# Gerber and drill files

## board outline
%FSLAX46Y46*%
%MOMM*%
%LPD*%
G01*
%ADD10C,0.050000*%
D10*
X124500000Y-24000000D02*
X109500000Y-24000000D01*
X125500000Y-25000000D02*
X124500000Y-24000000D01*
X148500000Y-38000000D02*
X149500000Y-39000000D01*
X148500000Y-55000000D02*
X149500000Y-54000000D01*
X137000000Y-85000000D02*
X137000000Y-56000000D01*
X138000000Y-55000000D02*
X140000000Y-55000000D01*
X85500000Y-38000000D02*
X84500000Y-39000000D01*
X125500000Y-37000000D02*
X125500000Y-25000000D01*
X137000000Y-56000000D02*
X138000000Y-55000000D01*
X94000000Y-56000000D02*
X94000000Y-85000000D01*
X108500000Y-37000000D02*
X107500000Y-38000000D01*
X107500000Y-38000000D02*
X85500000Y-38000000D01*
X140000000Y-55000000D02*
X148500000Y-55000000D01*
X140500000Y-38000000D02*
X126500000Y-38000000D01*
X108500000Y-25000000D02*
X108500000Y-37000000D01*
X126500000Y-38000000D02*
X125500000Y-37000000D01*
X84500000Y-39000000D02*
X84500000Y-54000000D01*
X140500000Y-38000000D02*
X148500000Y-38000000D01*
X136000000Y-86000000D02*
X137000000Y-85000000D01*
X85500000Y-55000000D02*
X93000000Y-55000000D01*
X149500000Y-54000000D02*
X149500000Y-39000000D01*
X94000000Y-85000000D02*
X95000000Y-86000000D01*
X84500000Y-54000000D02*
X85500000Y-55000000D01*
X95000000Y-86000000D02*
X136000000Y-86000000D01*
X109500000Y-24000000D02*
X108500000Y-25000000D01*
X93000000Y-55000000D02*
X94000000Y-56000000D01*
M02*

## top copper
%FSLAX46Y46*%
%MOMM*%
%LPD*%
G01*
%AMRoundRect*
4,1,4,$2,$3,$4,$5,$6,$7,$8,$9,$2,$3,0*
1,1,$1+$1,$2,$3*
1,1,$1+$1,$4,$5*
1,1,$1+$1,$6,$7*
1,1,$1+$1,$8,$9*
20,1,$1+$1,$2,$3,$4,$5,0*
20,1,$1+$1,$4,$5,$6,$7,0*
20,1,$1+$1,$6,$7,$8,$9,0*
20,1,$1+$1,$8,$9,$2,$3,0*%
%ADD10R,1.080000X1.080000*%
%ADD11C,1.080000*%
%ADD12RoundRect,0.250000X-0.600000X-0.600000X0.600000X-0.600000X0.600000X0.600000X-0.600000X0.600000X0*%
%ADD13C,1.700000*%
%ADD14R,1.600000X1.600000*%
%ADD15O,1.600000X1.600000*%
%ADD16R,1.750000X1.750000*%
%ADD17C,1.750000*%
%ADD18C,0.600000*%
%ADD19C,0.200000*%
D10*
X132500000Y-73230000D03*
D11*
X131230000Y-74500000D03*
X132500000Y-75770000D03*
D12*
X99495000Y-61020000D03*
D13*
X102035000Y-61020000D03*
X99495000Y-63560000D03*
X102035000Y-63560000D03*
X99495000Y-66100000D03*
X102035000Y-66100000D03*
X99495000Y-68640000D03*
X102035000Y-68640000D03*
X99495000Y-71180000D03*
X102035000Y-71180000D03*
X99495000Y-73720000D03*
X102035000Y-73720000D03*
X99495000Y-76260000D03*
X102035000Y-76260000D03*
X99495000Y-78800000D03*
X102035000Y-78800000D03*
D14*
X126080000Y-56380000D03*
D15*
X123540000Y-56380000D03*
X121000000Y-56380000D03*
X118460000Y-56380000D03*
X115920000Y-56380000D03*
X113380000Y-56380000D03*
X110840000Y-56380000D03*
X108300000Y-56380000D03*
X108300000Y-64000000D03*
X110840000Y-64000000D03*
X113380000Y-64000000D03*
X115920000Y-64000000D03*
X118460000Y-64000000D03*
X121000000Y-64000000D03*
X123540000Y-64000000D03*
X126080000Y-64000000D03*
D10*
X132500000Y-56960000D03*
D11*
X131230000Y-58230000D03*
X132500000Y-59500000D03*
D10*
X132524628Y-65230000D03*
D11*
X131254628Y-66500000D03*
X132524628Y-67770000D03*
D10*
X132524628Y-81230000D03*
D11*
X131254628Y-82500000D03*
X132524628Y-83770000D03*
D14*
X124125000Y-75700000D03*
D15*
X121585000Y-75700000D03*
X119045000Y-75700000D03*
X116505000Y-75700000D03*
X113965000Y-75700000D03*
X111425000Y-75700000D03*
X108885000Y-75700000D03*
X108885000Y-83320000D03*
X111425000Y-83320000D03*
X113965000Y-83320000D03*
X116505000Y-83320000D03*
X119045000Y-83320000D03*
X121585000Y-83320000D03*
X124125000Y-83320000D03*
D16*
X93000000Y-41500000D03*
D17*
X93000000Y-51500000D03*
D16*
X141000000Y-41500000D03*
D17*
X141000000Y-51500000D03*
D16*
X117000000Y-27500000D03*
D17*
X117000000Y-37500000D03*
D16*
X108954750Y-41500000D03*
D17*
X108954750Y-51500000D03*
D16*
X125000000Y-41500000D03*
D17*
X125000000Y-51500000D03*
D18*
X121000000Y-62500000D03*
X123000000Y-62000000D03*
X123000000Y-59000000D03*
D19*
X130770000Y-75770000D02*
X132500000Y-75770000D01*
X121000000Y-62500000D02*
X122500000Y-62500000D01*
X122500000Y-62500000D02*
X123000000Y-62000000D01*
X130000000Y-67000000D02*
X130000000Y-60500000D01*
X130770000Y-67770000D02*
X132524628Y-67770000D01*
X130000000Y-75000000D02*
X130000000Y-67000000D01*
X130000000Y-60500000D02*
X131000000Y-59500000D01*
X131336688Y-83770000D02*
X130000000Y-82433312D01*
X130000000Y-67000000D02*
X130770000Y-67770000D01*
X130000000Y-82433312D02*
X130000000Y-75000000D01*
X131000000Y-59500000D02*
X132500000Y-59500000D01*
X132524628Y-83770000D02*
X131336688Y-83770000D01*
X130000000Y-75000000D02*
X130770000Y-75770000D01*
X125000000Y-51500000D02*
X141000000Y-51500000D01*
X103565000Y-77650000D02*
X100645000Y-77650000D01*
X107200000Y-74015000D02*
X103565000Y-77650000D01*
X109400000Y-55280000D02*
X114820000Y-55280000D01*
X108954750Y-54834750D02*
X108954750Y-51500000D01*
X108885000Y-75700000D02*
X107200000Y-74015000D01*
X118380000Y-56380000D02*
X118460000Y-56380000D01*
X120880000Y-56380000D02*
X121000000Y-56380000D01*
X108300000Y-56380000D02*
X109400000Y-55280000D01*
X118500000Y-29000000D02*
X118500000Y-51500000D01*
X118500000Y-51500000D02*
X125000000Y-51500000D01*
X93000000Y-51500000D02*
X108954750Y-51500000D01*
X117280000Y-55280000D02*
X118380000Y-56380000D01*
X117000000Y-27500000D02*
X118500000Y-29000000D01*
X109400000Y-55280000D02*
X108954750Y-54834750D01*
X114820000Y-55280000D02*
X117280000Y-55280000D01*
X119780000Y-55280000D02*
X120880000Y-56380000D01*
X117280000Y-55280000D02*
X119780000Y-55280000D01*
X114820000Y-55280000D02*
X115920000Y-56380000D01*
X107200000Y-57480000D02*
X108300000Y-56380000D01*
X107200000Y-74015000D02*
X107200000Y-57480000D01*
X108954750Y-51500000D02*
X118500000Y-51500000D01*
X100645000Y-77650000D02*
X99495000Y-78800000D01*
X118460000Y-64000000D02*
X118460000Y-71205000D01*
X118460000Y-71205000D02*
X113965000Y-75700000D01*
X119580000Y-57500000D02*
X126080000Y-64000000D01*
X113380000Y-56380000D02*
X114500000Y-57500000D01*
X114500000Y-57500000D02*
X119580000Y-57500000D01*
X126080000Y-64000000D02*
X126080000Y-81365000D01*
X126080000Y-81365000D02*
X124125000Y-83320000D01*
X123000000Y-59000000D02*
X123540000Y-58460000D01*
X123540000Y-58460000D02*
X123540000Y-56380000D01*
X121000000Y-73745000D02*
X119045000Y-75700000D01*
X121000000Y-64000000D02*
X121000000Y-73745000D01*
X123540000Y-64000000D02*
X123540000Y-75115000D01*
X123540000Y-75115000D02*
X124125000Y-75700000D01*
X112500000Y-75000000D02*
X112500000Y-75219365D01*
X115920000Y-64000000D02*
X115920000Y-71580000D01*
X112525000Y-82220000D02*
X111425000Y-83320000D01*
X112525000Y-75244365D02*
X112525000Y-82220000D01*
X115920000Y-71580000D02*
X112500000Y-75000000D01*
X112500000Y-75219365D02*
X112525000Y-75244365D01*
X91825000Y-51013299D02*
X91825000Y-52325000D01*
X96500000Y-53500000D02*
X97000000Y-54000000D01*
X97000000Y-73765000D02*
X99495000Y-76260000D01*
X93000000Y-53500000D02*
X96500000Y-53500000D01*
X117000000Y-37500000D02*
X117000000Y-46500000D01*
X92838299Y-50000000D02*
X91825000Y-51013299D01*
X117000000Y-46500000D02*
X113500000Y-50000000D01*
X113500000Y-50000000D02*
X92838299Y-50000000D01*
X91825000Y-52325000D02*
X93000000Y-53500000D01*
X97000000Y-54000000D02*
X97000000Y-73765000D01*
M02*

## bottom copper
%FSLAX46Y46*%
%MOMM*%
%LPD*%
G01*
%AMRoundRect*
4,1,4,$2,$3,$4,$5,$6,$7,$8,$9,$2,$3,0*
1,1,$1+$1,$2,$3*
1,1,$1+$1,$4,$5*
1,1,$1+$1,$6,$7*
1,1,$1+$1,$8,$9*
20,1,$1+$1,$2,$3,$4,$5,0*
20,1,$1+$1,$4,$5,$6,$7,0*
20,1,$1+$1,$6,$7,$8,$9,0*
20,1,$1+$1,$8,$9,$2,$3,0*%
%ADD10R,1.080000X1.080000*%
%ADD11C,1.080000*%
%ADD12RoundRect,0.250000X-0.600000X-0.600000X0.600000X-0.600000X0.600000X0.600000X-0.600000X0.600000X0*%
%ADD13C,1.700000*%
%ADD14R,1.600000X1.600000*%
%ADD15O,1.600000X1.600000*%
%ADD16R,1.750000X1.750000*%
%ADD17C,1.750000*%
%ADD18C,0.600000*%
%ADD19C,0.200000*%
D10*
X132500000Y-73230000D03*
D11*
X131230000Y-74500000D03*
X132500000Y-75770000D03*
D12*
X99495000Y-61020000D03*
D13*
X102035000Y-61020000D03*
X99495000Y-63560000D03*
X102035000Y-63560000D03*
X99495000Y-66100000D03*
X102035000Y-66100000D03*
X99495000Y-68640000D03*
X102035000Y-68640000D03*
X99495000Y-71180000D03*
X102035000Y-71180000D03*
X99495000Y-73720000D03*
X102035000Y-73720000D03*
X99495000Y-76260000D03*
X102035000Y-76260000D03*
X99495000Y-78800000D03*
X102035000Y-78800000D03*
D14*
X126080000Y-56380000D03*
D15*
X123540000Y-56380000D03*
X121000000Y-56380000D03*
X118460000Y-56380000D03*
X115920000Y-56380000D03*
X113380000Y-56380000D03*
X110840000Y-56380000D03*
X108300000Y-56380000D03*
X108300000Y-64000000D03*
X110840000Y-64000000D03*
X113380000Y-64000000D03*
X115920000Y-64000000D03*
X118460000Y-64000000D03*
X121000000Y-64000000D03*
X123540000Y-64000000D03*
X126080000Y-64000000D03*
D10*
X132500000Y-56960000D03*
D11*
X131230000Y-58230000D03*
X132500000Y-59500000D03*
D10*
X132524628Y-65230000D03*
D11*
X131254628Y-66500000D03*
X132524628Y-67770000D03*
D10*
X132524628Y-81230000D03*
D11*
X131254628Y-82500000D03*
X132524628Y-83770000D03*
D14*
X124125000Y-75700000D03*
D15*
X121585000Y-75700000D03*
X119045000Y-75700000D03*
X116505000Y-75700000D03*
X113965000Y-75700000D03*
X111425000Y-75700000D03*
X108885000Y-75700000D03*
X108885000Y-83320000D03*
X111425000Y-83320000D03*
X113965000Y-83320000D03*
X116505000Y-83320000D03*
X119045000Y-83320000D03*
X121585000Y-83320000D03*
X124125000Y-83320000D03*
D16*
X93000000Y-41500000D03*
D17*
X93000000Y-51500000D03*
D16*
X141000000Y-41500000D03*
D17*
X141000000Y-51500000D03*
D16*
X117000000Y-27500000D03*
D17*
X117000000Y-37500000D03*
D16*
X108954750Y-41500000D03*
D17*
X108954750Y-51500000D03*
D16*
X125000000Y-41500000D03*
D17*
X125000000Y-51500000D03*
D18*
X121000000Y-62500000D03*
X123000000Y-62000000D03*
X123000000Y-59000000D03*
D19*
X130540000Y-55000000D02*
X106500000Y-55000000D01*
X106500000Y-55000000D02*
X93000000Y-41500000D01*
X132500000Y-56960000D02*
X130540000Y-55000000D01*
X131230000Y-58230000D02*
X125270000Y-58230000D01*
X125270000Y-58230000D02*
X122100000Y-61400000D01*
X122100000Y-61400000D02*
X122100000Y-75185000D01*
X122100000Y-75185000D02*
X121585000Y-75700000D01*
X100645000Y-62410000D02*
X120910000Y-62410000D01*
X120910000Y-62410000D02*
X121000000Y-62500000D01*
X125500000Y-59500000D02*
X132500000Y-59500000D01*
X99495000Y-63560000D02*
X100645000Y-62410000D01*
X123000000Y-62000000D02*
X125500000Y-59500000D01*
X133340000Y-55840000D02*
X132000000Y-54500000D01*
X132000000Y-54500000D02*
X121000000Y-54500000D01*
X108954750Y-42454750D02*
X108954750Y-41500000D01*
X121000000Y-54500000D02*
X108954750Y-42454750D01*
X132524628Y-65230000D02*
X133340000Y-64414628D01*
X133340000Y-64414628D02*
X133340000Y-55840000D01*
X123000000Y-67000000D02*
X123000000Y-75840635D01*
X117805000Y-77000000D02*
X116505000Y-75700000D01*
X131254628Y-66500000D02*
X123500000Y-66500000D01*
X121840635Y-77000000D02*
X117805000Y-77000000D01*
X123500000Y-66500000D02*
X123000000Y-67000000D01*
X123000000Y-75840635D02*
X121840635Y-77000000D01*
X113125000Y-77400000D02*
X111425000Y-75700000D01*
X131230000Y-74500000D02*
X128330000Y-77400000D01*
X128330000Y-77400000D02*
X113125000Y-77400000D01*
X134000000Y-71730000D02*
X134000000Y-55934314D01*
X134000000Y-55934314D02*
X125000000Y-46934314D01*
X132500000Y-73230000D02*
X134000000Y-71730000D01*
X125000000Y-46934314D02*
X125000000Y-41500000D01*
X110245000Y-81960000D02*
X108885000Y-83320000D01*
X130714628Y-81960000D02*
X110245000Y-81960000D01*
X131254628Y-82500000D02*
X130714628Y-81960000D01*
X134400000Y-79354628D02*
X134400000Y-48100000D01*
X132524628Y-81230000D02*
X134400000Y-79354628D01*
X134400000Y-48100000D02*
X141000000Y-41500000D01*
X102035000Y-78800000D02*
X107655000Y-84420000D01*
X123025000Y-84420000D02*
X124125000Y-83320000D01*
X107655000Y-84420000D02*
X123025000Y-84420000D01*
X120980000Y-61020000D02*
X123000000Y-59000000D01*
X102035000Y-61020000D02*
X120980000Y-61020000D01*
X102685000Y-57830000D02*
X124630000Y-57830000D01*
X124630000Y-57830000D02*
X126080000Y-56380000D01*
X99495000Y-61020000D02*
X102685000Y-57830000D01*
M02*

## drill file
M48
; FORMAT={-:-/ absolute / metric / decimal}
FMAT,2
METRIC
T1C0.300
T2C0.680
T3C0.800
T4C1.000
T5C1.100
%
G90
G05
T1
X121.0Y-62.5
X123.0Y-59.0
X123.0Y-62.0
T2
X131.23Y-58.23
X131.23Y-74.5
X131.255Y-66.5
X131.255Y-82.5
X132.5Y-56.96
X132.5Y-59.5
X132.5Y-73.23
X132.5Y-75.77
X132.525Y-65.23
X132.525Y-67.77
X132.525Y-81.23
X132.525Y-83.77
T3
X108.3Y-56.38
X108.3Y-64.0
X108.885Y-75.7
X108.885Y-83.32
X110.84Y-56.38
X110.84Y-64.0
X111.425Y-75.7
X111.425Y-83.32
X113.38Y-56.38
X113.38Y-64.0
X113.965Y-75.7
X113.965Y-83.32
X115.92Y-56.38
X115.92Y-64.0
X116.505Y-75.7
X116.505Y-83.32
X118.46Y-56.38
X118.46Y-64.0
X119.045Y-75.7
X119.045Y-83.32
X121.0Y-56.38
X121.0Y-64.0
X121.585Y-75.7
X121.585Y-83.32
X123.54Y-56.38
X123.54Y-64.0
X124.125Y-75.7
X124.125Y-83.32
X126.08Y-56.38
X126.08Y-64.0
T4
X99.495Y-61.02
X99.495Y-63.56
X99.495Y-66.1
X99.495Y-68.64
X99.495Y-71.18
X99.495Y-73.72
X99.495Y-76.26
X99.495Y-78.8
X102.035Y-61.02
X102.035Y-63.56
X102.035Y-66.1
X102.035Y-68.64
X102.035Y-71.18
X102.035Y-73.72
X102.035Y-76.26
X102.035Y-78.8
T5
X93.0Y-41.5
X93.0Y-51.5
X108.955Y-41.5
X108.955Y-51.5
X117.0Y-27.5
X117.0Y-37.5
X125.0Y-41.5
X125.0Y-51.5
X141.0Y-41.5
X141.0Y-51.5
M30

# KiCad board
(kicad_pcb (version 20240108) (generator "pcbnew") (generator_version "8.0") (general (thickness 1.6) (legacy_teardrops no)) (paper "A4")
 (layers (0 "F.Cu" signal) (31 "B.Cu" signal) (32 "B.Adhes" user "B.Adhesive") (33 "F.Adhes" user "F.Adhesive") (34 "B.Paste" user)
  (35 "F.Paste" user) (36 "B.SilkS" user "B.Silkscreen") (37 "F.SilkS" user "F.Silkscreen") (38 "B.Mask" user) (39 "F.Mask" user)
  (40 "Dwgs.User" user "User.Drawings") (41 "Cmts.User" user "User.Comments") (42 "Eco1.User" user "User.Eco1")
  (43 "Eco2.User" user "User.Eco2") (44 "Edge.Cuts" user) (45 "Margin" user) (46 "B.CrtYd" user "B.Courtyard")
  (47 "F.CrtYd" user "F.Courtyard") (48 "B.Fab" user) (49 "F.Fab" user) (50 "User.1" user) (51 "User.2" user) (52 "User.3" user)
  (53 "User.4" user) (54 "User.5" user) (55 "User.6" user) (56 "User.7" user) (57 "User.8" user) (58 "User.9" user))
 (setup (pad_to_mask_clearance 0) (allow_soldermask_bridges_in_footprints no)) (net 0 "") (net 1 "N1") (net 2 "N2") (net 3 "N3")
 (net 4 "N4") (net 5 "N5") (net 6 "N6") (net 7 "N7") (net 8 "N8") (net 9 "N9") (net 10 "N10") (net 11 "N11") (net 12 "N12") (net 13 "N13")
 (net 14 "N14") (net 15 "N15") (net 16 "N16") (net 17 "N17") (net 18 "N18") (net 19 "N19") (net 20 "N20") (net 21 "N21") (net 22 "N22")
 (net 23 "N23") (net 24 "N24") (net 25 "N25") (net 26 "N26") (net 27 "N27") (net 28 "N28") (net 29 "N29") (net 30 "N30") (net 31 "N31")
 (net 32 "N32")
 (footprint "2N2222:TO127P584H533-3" (layer "F.Cu") (at 132.5 74.5 -90)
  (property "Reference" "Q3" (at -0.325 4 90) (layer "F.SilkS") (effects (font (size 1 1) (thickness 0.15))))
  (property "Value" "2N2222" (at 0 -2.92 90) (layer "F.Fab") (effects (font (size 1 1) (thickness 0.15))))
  (pad "1" thru_hole rect (at -1.27 0 270) (size 1.08 1.08) (drill 0.68) (layers "*.Cu" "*.Mask") (remove_unused_layers no) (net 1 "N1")
   (solder_mask_margin 0.102))
  (pad "2" thru_hole circle (at 0 1.27 270) (size 1.08 1.08) (drill 0.68) (layers "*.Cu" "*.Mask") (remove_unused_layers no) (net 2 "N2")
   (solder_mask_margin 0.102))
  (pad "3" thru_hole circle (at 1.27 0 267) (size 1.08 1.08) (drill 0.68) (layers "*.Cu" "*.Mask") (remove_unused_layers no) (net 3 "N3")
   (solder_mask_margin 0.102)))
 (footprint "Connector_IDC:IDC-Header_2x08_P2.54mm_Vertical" (layer "F.Cu") (at 99.495 61.02)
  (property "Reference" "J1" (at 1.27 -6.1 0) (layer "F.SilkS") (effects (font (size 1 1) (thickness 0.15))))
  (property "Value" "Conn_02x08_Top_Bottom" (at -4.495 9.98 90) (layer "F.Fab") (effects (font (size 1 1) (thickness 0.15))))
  (pad "1" thru_hole roundrect (at 0 0) (size 1.7 1.7) (drill 1) (layers "*.Cu" "*.Mask") (remove_unused_layers no)
   (roundrect_rratio 0.147059) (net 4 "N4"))
  (pad "2" thru_hole circle (at 2.54 0) (size 1.7 1.7) (drill 1) (layers "*.Cu" "*.Mask") (remove_unused_layers no) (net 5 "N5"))
  (pad "3" thru_hole circle (at 0 2.54) (size 1.7 1.7) (drill 1) (layers "*.Cu" "*.Mask") (remove_unused_layers no) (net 3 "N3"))
  (pad "4" thru_hole circle (at 2.54 2.54) (size 1.7 1.7) (drill 1) (layers "*.Cu" "*.Mask") (remove_unused_layers no) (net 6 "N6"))
  (pad "5" thru_hole circle (at 0 5.08) (size 1.7 1.7) (drill 1) (layers "*.Cu" "*.Mask") (remove_unused_layers no) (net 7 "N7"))
  (pad "6" thru_hole circle (at 2.54 5.08) (size 1.7 1.7) (drill 1) (layers "*.Cu" "*.Mask") (remove_unused_layers no) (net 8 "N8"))
  (pad "7" thru_hole circle (at 0 7.62) (size 1.7 1.7) (drill 1) (layers "*.Cu" "*.Mask") (remove_unused_layers no) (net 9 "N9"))
  (pad "8" thru_hole circle (at 2.54 7.62) (size 1.7 1.7) (drill 1) (layers "*.Cu" "*.Mask") (remove_unused_layers no) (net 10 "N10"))
  (pad "9" thru_hole circle (at 0 10.16) (size 1.7 1.7) (drill 1) (layers "*.Cu" "*.Mask") (remove_unused_layers no) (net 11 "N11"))
  (pad "10" thru_hole circle (at 2.54 10.16) (size 1.7 1.7) (drill 1) (layers "*.Cu" "*.Mask") (remove_unused_layers no) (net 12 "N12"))
  (pad "11" thru_hole circle (at 0 12.7) (size 1.7 1.7) (drill 1) (layers "*.Cu" "*.Mask") (remove_unused_layers no) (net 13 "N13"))
  (pad "12" thru_hole circle (at 2.54 12.7) (size 1.7 1.7) (drill 1) (layers "*.Cu" "*.Mask") (remove_unused_layers no) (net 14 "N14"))
  (pad "13" thru_hole circle (at 0 15.24) (size 1.7 1.7) (drill 1) (layers "*.Cu" "*.Mask") (remove_unused_layers no) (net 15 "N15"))
  (pad "14" thru_hole circle (at 2.54 15.24) (size 1.7 1.7) (drill 1) (layers "*.Cu" "*.Mask") (remove_unused_layers no) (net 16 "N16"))
  (pad "15" thru_hole circle (at 0 17.78) (size 1.7 1.7) (drill 1) (layers "*.Cu" "*.Mask") (remove_unused_layers no) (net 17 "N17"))
  (pad "16" thru_hole circle (at 2.54 17.78) (size 1.7 1.7) (drill 1) (layers "*.Cu" "*.Mask") (remove_unused_layers no) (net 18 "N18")))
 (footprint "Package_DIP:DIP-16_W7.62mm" (layer "F.Cu") (at 126.08 56.38 -90)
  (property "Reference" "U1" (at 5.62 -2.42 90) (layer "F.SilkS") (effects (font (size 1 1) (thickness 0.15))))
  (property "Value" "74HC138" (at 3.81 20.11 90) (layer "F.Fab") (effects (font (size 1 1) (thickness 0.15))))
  (pad "1" thru_hole rect (at 0 0 270) (size 1.6 1.6) (drill 0.8) (layers "*.Cu" "*.Mask") (remove_unused_layers no) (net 4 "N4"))
  (pad "2" thru_hole oval (at 0 2.54 270) (size 1.6 1.6) (drill 0.8) (layers "*.Cu" "*.Mask") (remove_unused_layers no) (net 5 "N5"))
  (pad "3" thru_hole oval (at 0 5.08 270) (size 1.6 1.6) (drill 0.8) (layers "*.Cu" "*.Mask") (remove_unused_layers no) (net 17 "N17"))
  (pad "4" thru_hole oval (at 0 7.62 270) (size 1.6 1.6) (drill 0.8) (layers "*.Cu" "*.Mask") (remove_unused_layers no) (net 17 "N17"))
  (pad "5" thru_hole oval (at 0 10.16 270) (size 1.6 1.6) (drill 0.8) (layers "*.Cu" "*.Mask") (remove_unused_layers no) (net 17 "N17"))
  (pad "6" thru_hole oval (at 0 12.7 270) (size 1.6 1.6) (drill 0.8) (layers "*.Cu" "*.Mask") (remove_unused_layers no) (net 18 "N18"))
  (pad "7" thru_hole oval (at 0 15.24 270) (size 1.6 1.6) (drill 0.8) (layers "*.Cu" "*.Mask") (remove_unused_layers no) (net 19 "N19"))
  (pad "8" thru_hole oval (at 0 17.78 270) (size 1.6 1.6) (drill 0.8) (layers "*.Cu" "*.Mask") (remove_unused_layers no) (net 17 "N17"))
  (pad "9" thru_hole oval (at 7.62 17.78 270) (size 1.6 1.6) (drill 0.8) (layers "*.Cu" "*.Mask") (remove_unused_layers no) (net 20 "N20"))
  (pad "10" thru_hole oval (at 7.62 15.24 270) (size 1.6 1.6) (drill 0.8) (layers "*.Cu" "*.Mask") (remove_unused_layers no) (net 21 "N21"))
  (pad "11" thru_hole oval (at 7.62 12.7 270) (size 1.6 1.6) (drill 0.8) (layers "*.Cu" "*.Mask") (remove_unused_layers no) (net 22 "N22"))
  (pad "12" thru_hole oval (at 7.62 10.16 270) (size 1.6 1.6) (drill 0.8) (layers "*.Cu" "*.Mask") (remove_unused_layers no) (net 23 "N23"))
  (pad "13" thru_hole oval (at 7.62 7.62 270) (size 1.6 1.6) (drill 0.8) (layers "*.Cu" "*.Mask") (remove_unused_layers no) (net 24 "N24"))
  (pad "14" thru_hole oval (at 7.62 5.08 270) (size 1.6 1.6) (drill 0.8) (layers "*.Cu" "*.Mask") (remove_unused_layers no) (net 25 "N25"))
  (pad "15" thru_hole oval (at 7.62 2.54 270) (size 1.6 1.6) (drill 0.8) (layers "*.Cu" "*.Mask") (remove_unused_layers no) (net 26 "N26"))
  (pad "16" thru_hole oval (at 7.62 0 270) (size 1.6 1.6) (drill 0.8) (layers "*.Cu" "*.Mask") (remove_unused_layers no) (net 18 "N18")))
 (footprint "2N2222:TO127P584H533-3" (layer "F.Cu") (at 132.5 58.23 -90)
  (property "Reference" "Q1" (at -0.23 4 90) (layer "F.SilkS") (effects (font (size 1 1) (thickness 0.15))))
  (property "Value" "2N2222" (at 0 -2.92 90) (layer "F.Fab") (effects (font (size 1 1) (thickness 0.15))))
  (pad "1" thru_hole rect (at -1.27 0 270) (size 1.08 1.08) (drill 0.68) (layers "*.Cu" "*.Mask") (remove_unused_layers no) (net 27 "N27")
   (solder_mask_margin 0.102))
  (pad "2" thru_hole circle (at 0 1.27 270) (size 1.08 1.08) (drill 0.68) (layers "*.Cu" "*.Mask") (remove_unused_layers no) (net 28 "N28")
   (solder_mask_margin 0.102))
  (pad "3" thru_hole circle (at 1.27 0 267) (size 1.08 1.08) (drill 0.68) (layers "*.Cu" "*.Mask") (remove_unused_layers no) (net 3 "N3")
   (solder_mask_margin 0.102)))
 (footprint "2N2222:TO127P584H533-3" (layer "F.Cu") (at 132.524628 66.5 -90)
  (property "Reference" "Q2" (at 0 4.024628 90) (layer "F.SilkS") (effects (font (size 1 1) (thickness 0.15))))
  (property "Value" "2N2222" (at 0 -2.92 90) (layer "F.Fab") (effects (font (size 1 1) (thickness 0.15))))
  (pad "1" thru_hole rect (at -1.27 0 270) (size 1.08 1.08) (drill 0.68) (layers "*.Cu" "*.Mask") (remove_unused_layers no) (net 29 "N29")
   (solder_mask_margin 0.102))
  (pad "2" thru_hole circle (at 0 1.27 270) (size 1.08 1.08) (drill 0.68) (layers "*.Cu" "*.Mask") (remove_unused_layers no) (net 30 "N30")
   (solder_mask_margin 0.102))
  (pad "3" thru_hole circle (at 1.27 0 267) (size 1.08 1.08) (drill 0.68) (layers "*.Cu" "*.Mask") (remove_unused_layers no) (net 3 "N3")
   (solder_mask_margin 0.102)))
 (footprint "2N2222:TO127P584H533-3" (layer "F.Cu") (at 132.524628 82.5 -90)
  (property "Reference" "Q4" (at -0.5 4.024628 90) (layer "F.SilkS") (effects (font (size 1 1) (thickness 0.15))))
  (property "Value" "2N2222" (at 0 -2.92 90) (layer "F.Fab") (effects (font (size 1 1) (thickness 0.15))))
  (pad "1" thru_hole rect (at -1.27 0 270) (size 1.08 1.08) (drill 0.68) (layers "*.Cu" "*.Mask") (remove_unused_layers no) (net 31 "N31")
   (solder_mask_margin 0.102))
  (pad "2" thru_hole circle (at 0 1.27 270) (size 1.08 1.08) (drill 0.68) (layers "*.Cu" "*.Mask") (remove_unused_layers no) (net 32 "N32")
   (solder_mask_margin 0.102))
  (pad "3" thru_hole circle (at 1.27 0 267) (size 1.08 1.08) (drill 0.68) (layers "*.Cu" "*.Mask") (remove_unused_layers no) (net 3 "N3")
   (solder_mask_margin 0.102)))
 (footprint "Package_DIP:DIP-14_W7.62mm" (layer "F.Cu") (at 124.125 75.7 -90)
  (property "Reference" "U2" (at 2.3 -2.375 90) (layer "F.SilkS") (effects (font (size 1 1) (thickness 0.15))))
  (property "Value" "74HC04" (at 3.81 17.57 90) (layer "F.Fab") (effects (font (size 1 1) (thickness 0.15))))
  (pad "1" thru_hole rect (at 0 0 270) (size 1.6 1.6) (drill 0.8) (layers "*.Cu" "*.Mask") (remove_unused_layers no) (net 26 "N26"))
  (pad "2" thru_hole oval (at 0 2.54 270) (size 1.6 1.6) (drill 0.8) (layers "*.Cu" "*.Mask") (remove_unused_layers no) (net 28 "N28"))
  (pad "3" thru_hole oval (at 0 5.08 270) (size 1.6 1.6) (drill 0.8) (layers "*.Cu" "*.Mask") (remove_unused_layers no) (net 25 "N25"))
  (pad "4" thru_hole oval (at 0 7.62 270) (size 1.6 1.6) (drill 0.8) (layers "*.Cu" "*.Mask") (remove_unused_layers no) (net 30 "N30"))
  (pad "5" thru_hole oval (at 0 10.16 270) (size 1.6 1.6) (drill 0.8) (layers "*.Cu" "*.Mask") (remove_unused_layers no) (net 24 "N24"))
  (pad "6" thru_hole oval (at 0 12.7 270) (size 1.6 1.6) (drill 0.8) (layers "*.Cu" "*.Mask") (remove_unused_layers no) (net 2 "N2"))
  (pad "7" thru_hole oval (at 0 15.24 270) (size 1.6 1.6) (drill 0.8) (layers "*.Cu" "*.Mask") (remove_unused_layers no) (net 17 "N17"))
  (pad "8" thru_hole oval (at 7.62 15.24 270) (size 1.6 1.6) (drill 0.8) (layers "*.Cu" "*.Mask") (remove_unused_layers no) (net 32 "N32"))
  (pad "9" thru_hole oval (at 7.62 12.7 270) (size 1.6 1.6) (drill 0.8) (layers "*.Cu" "*.Mask") (remove_unused_layers no) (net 23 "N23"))
  (pad "10" thru_hole oval (at 7.62 10.16 270) (size 1.6 1.6) (drill 0.8) (layers "*.Cu" "*.Mask") (remove_unused_layers no))
  (pad "11" thru_hole oval (at 7.62 7.62 270) (size 1.6 1.6) (drill 0.8) (layers "*.Cu" "*.Mask") (remove_unused_layers no))
  (pad "12" thru_hole oval (at 7.62 5.08 270) (size 1.6 1.6) (drill 0.8) (layers "*.Cu" "*.Mask") (remove_unused_layers no))
  (pad "13" thru_hole oval (at 7.62 2.54 270) (size 1.6 1.6) (drill 0.8) (layers "*.Cu" "*.Mask") (remove_unused_layers no))
  (pad "14" thru_hole oval (at 7.62 0 270) (size 1.6 1.6) (drill 0.8) (layers "*.Cu" "*.Mask") (remove_unused_layers no) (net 18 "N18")))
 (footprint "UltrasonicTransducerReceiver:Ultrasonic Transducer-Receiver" (layer "B.Cu") (at 93 41.5 -90)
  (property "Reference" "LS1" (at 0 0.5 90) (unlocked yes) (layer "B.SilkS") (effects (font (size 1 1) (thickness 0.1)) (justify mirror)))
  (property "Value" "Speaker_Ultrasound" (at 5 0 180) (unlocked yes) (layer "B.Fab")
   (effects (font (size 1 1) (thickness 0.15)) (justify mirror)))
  (pad "1" thru_hole rect (at 0 0 270) (size 1.75 1.75) (drill 1.1) (layers "*.Cu" "*.Mask") (remove_unused_layers no) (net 27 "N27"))
  (pad "2" thru_hole circle (at 10 0 270) (size 1.75 1.75) (drill 1.1) (layers "*.Cu" "*.Mask") (remove_unused_layers no) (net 17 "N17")))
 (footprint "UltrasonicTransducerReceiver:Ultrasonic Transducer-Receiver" (layer "B.Cu") (at 141 41.5 -90)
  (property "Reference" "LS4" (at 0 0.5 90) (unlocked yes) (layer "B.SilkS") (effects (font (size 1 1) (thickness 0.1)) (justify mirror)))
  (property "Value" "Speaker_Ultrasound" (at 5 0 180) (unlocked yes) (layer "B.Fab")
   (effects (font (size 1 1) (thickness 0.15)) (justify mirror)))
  (pad "1" thru_hole rect (at 0 0 270) (size 1.75 1.75) (drill 1.1) (layers "*.Cu" "*.Mask") (remove_unused_layers no) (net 31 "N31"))
  (pad "2" thru_hole circle (at 10 0 270) (size 1.75 1.75) (drill 1.1) (layers "*.Cu" "*.Mask") (remove_unused_layers no) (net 17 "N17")))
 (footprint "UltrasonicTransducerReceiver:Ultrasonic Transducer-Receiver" (layer "B.Cu") (at 117 27.5 -90)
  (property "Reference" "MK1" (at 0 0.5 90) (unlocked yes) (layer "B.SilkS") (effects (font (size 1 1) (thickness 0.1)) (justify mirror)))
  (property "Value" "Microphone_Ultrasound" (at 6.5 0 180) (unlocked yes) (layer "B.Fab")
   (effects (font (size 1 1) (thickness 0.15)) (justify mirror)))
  (pad "1" thru_hole rect (at 0 0 270) (size 1.75 1.75) (drill 1.1) (layers "*.Cu" "*.Mask") (remove_unused_layers no) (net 17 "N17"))
  (pad "2" thru_hole circle (at 10 0 270) (size 1.75 1.75) (drill 1.1) (layers "*.Cu" "*.Mask") (remove_unused_layers no) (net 15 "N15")))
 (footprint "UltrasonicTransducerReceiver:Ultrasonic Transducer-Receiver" (layer "B.Cu") (at 108.95475 41.5 -90)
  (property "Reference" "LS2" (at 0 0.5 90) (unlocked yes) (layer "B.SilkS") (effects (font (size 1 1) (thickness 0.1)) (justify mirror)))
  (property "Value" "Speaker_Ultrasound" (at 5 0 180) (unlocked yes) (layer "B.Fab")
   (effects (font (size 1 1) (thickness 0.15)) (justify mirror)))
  (pad "1" thru_hole rect (at 0 0 270) (size 1.75 1.75) (drill 1.1) (layers "*.Cu" "*.Mask") (remove_unused_layers no) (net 29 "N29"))
  (pad "2" thru_hole circle (at 10 0 270) (size 1.75 1.75) (drill 1.1) (layers "*.Cu" "*.Mask") (remove_unused_layers no) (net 17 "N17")))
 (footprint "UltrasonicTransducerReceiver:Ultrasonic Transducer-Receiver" (layer "B.Cu") (at 125 41.5 -90)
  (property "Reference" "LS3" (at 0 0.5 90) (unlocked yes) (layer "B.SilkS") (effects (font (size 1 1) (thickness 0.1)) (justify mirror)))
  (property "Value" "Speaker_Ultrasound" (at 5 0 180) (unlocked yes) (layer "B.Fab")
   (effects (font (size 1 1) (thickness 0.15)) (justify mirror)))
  (pad "1" thru_hole rect (at 0 0 270) (size 1.75 1.75) (drill 1.1) (layers "*.Cu" "*.Mask") (remove_unused_layers no) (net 1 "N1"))
  (pad "2" thru_hole circle (at 10 0 270) (size 1.75 1.75) (drill 1.1) (layers "*.Cu" "*.Mask") (remove_unused_layers no) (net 17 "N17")))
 (gr_line (start 124.5 24) (end 109.5 24) (stroke (width 0.05) (type default)) (layer "Edge.Cuts"))
 (gr_line (start 125.5 25) (end 124.5 24) (stroke (width 0.05) (type default)) (layer "Edge.Cuts"))
 (gr_line (start 148.5 38) (end 149.5 39) (stroke (width 0.05) (type default)) (layer "Edge.Cuts"))
 (gr_line (start 148.5 55) (end 149.5 54) (stroke (width 0.05) (type default)) (layer "Edge.Cuts"))
 (gr_line (start 137 85) (end 137 56) (stroke (width 0.05) (type default)) (layer "Edge.Cuts"))
 (gr_line (start 138 55) (end 140 55) (stroke (width 0.05) (type default)) (layer "Edge.Cuts"))
 (gr_line (start 85.5 38) (end 84.5 39) (stroke (width 0.05) (type default)) (layer "Edge.Cuts"))
 (gr_line (start 125.5 37) (end 125.5 25) (stroke (width 0.05) (type default)) (layer "Edge.Cuts"))
 (gr_line (start 137 56) (end 138 55) (stroke (width 0.05) (type default)) (layer "Edge.Cuts"))
 (gr_line (start 94 56) (end 94 85) (stroke (width 0.05) (type default)) (layer "Edge.Cuts"))
 (gr_line (start 108.5 37) (end 107.5 38) (stroke (width 0.05) (type default)) (layer "Edge.Cuts"))
 (gr_line (start 107.5 38) (end 85.5 38) (stroke (width 0.05) (type default)) (layer "Edge.Cuts"))
 (gr_line (start 140 55) (end 148.5 55) (stroke (width 0.05) (type default)) (layer "Edge.Cuts"))
 (gr_line (start 140.5 38) (end 126.5 38) (stroke (width 0.05) (type default)) (layer "Edge.Cuts"))
 (gr_line (start 108.5 25) (end 108.5 37) (stroke (width 0.05) (type default)) (layer "Edge.Cuts"))
 (gr_line (start 126.5 38) (end 125.5 37) (stroke (width 0.05) (type default)) (layer "Edge.Cuts"))
 (gr_line (start 84.5 39) (end 84.5 54) (stroke (width 0.05) (type default)) (layer "Edge.Cuts"))
 (gr_line (start 140.5 38) (end 148.5 38) (stroke (width 0.05) (type default)) (layer "Edge.Cuts"))
 (gr_line (start 136 86) (end 137 85) (stroke (width 0.05) (type default)) (layer "Edge.Cuts"))
 (gr_line (start 85.5 55) (end 93 55) (stroke (width 0.05) (type default)) (layer "Edge.Cuts"))
 (gr_line (start 149.5 54) (end 149.5 39) (stroke (width 0.05) (type default)) (layer "Edge.Cuts"))
 (gr_line (start 94 85) (end 95 86) (stroke (width 0.05) (type default)) (layer "Edge.Cuts"))
 (gr_line (start 84.5 54) (end 85.5 55) (stroke (width 0.05) (type default)) (layer "Edge.Cuts"))
 (gr_line (start 95 86) (end 136 86) (stroke (width 0.05) (type default)) (layer "Edge.Cuts"))
 (gr_line (start 109.5 24) (end 108.5 25) (stroke (width 0.05) (type default)) (layer "Edge.Cuts"))
 (gr_line (start 93 55) (end 94 56) (stroke (width 0.05) (type default)) (layer "Edge.Cuts"))
 (segment (start 130.54 55) (end 106.5 55) (width 0.2) (layer "B.Cu") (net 27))
 (segment (start 106.5 55) (end 93 41.5) (width 0.2) (layer "B.Cu") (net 27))
 (segment (start 132.5 56.96) (end 130.54 55) (width 0.2) (layer "B.Cu") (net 27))
 (segment (start 131.23 58.23) (end 125.27 58.23) (width 0.2) (layer "B.Cu") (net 28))
 (segment (start 125.27 58.23) (end 122.1 61.4) (width 0.2) (layer "B.Cu") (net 28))
 (segment (start 122.1 61.4) (end 122.1 75.185) (width 0.2) (layer "B.Cu") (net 28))
 (segment (start 122.1 75.185) (end 121.585 75.7) (width 0.2) (layer "B.Cu") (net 28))
 (segment (start 130.77 75.77) (end 132.5 75.77) (width 0.2) (layer "F.Cu") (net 3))
 (segment (start 121 62.5) (end 122.5 62.5) (width 0.2) (layer "F.Cu") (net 3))
 (segment (start 122.5 62.5) (end 123 62) (width 0.2) (layer "F.Cu") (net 3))
 (segment (start 130 67) (end 130 60.5) (width 0.2) (layer "F.Cu") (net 3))
 (segment (start 130.77 67.77) (end 132.524628 67.77) (width 0.2) (layer "F.Cu") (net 3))
 (segment (start 130 75) (end 130 67) (width 0.2) (layer "F.Cu") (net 3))
 (segment (start 130 60.5) (end 131 59.5) (width 0.2) (layer "F.Cu") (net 3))
 (segment (start 131.336688 83.77) (end 130 82.433312) (width 0.2) (layer "F.Cu") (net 3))
 (segment (start 130 67) (end 130.77 67.77) (width 0.2) (layer "F.Cu") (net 3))
 (segment (start 130 82.433312) (end 130 75) (width 0.2) (layer "F.Cu") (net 3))
 (segment (start 131 59.5) (end 132.5 59.5) (width 0.2) (layer "F.Cu") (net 3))
 (segment (start 132.524628 83.77) (end 131.336688 83.77) (width 0.2) (layer "F.Cu") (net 3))
 (segment (start 130 75) (end 130.77 75.77) (width 0.2) (layer "F.Cu") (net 3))
 (via (at 121 62.5) (size 0.6) (drill 0.3) (layers "F.Cu" "B.Cu") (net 3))
 (via (at 123 62) (size 0.6) (drill 0.3) (layers "F.Cu" "B.Cu") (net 3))
 (segment (start 100.645 62.41) (end 120.91 62.41) (width 0.2) (layer "B.Cu") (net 3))
 (segment (start 120.91 62.41) (end 121 62.5) (width 0.2) (layer "B.Cu") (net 3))
 (segment (start 125.5 59.5) (end 132.5 59.5) (width 0.2) (layer "B.Cu") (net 3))
 (segment (start 99.495 63.56) (end 100.645 62.41) (width 0.2) (layer "B.Cu") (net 3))
 (segment (start 123 62) (end 125.5 59.5) (width 0.2) (layer "B.Cu") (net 3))
 (segment (start 133.34 55.84) (end 132 54.5) (width 0.2) (layer "B.Cu") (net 29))
 (segment (start 132 54.5) (end 121 54.5) (width 0.2) (layer "B.Cu") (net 29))
 (segment (start 108.95475 42.45475) (end 108.95475 41.5) (width 0.2) (layer "B.Cu") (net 29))
 (segment (start 121 54.5) (end 108.95475 42.45475) (width 0.2) (layer "B.Cu") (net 29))
 (segment (start 132.524628 65.23) (end 133.34 64.414628) (width 0.2) (layer "B.Cu") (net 29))
 (segment (start 133.34 64.414628) (end 133.34 55.84) (width 0.2) (layer "B.Cu") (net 29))
 (segment (start 123 67) (end 123 75.840635) (width 0.2) (layer "B.Cu") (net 30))
 (segment (start 117.805 77) (end 116.505 75.7) (width 0.2) (layer "B.Cu") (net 30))
 (segment (start 131.254628 66.5) (end 123.5 66.5) (width 0.2) (layer "B.Cu") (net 30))
 (segment (start 121.840635 77) (end 117.805 77) (width 0.2) (layer "B.Cu") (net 30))
 (segment (start 123.5 66.5) (end 123 67) (width 0.2) (layer "B.Cu") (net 30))
 (segment (start 123 75.840635) (end 121.840635 77) (width 0.2) (layer "B.Cu") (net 30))
 (segment (start 113.125 77.4) (end 111.425 75.7) (width 0.2) (layer "B.Cu") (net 2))
 (segment (start 131.23 74.5) (end 128.33 77.4) (width 0.2) (layer "B.Cu") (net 2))
 (segment (start 128.33 77.4) (end 113.125 77.4) (width 0.2) (layer "B.Cu") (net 2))
 (segment (start 134 71.73) (end 134 55.934314) (width 0.2) (layer "B.Cu") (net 1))
 (segment (start 134 55.934314) (end 125 46.934314) (width 0.2) (layer "B.Cu") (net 1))
 (segment (start 132.5 73.23) (end 134 71.73) (width 0.2) (layer "B.Cu") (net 1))
 (segment (start 125 46.934314) (end 125 41.5) (width 0.2) (layer "B.Cu") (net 1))
 (segment (start 110.245 81.96) (end 108.885 83.32) (width 0.2) (layer "B.Cu") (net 32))
 (segment (start 130.714628 81.96) (end 110.245 81.96) (width 0.2) (layer "B.Cu") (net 32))
 (segment (start 131.254628 82.5) (end 130.714628 81.96) (width 0.2) (layer "B.Cu") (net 32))
 (segment (start 134.4 79.354628) (end 134.4 48.1) (width 0.2) (layer "B.Cu") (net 31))
 (segment (start 132.524628 81.23) (end 134.4 79.354628) (width 0.2) (layer "B.Cu") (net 31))
 (segment (start 134.4 48.1) (end 141 41.5) (width 0.2) (layer "B.Cu") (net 31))
 (segment (start 125 51.5) (end 141 51.5) (width 0.2) (layer "F.Cu") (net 17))
 (segment (start 103.565 77.65) (end 100.645 77.65) (width 0.2) (layer "F.Cu") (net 17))
 (segment (start 107.2 74.015) (end 103.565 77.65) (width 0.2) (layer "F.Cu") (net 17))
 (segment (start 109.4 55.28) (end 114.82 55.28) (width 0.2) (layer "F.Cu") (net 17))
 (segment (start 108.95475 54.83475) (end 108.95475 51.5) (width 0.2) (layer "F.Cu") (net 17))
 (segment (start 108.885 75.7) (end 107.2 74.015) (width 0.2) (layer "F.Cu") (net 17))
 (segment (start 118.38 56.38) (end 118.46 56.38) (width 0.2) (layer "F.Cu") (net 17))
 (segment (start 120.88 56.38) (end 121 56.38) (width 0.2) (layer "F.Cu") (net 17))
 (segment (start 108.3 56.38) (end 109.4 55.28) (width 0.2) (layer "F.Cu") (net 17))
 (segment (start 118.5 29) (end 118.5 51.5) (width 0.2) (layer "F.Cu") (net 17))
 (segment (start 118.5 51.5) (end 125 51.5) (width 0.2) (layer "F.Cu") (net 17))
 (segment (start 93 51.5) (end 108.95475 51.5) (width 0.2) (layer "F.Cu") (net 17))
 (segment (start 117.28 55.28) (end 118.38 56.38) (width 0.2) (layer "F.Cu") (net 17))
 (segment (start 117 27.5) (end 118.5 29) (width 0.2) (layer "F.Cu") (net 17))
 (segment (start 109.4 55.28) (end 108.95475 54.83475) (width 0.2) (layer "F.Cu") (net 17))
 (segment (start 114.82 55.28) (end 117.28 55.28) (width 0.2) (layer "F.Cu") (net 17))
 (segment (start 119.78 55.28) (end 120.88 56.38) (width 0.2) (layer "F.Cu") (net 17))
 (segment (start 117.28 55.28) (end 119.78 55.28) (width 0.2) (layer "F.Cu") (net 17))
 (segment (start 114.82 55.28) (end 115.92 56.38) (width 0.2) (layer "F.Cu") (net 17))
 (segment (start 107.2 57.48) (end 108.3 56.38) (width 0.2) (layer "F.Cu") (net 17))
 (segment (start 107.2 74.015) (end 107.2 57.48) (width 0.2) (layer "F.Cu") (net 17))
 (segment (start 108.95475 51.5) (end 118.5 51.5) (width 0.2) (layer "F.Cu") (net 17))
 (segment (start 100.645 77.65) (end 99.495 78.8) (width 0.2) (layer "F.Cu") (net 17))
 (segment (start 118.46 64) (end 118.46 71.205) (width 0.2) (layer "F.Cu") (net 24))
 (segment (start 118.46 71.205) (end 113.965 75.7) (width 0.2) (layer "F.Cu") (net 24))
 (segment (start 119.58 57.5) (end 126.08 64) (width 0.2) (layer "F.Cu") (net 18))
 (segment (start 113.38 56.38) (end 114.5 57.5) (width 0.2) (layer "F.Cu") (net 18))
 (segment (start 114.5 57.5) (end 119.58 57.5) (width 0.2) (layer "F.Cu") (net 18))
 (segment (start 126.08 64) (end 126.08 81.365) (width 0.2) (layer "F.Cu") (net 18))
 (segment (start 126.08 81.365) (end 124.125 83.32) (width 0.2) (layer "F.Cu") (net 18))
 (segment (start 102.035 78.8) (end 107.655 84.42) (width 0.2) (layer "B.Cu") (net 18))
 (segment (start 123.025 84.42) (end 124.125 83.32) (width 0.2) (layer "B.Cu") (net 18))
 (segment (start 107.655 84.42) (end 123.025 84.42) (width 0.2) (layer "B.Cu") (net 18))
 (segment (start 123 59) (end 123.54 58.46) (width 0.2) (layer "F.Cu") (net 5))
 (segment (start 123.54 58.46) (end 123.54 56.38) (width 0.2) (layer "F.Cu") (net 5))
 (via (at 123 59) (size 0.6) (drill 0.3) (layers "F.Cu" "B.Cu") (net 5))
 (segment (start 120.98 61.02) (end 123 59) (width 0.2) (layer "B.Cu") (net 5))
 (segment (start 102.035 61.02) (end 120.98 61.02) (width 0.2) (layer "B.Cu") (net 5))
 (segment (start 121 73.745) (end 119.045 75.7) (width 0.2) (layer "F.Cu") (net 25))
 (segment (start 121 64) (end 121 73.745) (width 0.2) (layer "F.Cu") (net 25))
 (segment (start 123.54 64) (end 123.54 75.115) (width 0.2) (layer "F.Cu") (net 26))
 (segment (start 123.54 75.115) (end 124.125 75.7) (width 0.2) (layer "F.Cu") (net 26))
 (segment (start 102.685 57.83) (end 124.63 57.83) (width 0.2) (layer "B.Cu") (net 4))
 (segment (start 124.63 57.83) (end 126.08 56.38) (width 0.2) (layer "B.Cu") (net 4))
 (segment (start 99.495 61.02) (end 102.685 57.83) (width 0.2) (layer "B.Cu") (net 4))
 (segment (start 112.5 75) (end 112.5 75.219365) (width 0.2) (layer "F.Cu") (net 23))
 (segment (start 115.92 64) (end 115.92 71.58) (width 0.2) (layer "F.Cu") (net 23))
 (segment (start 112.525 82.22) (end 111.425 83.32) (width 0.2) (layer "F.Cu") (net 23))
 (segment (start 112.525 75.244365) (end 112.525 82.22) (width 0.2) (layer "F.Cu") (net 23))
 (segment (start 115.92 71.58) (end 112.5 75) (width 0.2) (layer "F.Cu") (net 23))
 (segment (start 112.5 75.219365) (end 112.525 75.244365) (width 0.2) (layer "F.Cu") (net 23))
 (segment (start 91.825 51.013299) (end 91.825 52.325) (width 0.2) (layer "F.Cu") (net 15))
 (segment (start 96.5 53.5) (end 97 54) (width 0.2) (layer "F.Cu") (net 15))
 (segment (start 97 73.765) (end 99.495 76.26) (width 0.2) (layer "F.Cu") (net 15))
 (segment (start 93 53.5) (end 96.5 53.5) (width 0.2) (layer "F.Cu") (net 15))
 (segment (start 117 37.5) (end 117 46.5) (width 0.2) (layer "F.Cu") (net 15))
 (segment (start 92.838299 50) (end 91.825 51.013299) (width 0.2) (layer "F.Cu") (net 15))
 (segment (start 117 46.5) (end 113.5 50) (width 0.2) (layer "F.Cu") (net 15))
 (segment (start 113.5 50) (end 92.838299 50) (width 0.2) (layer "F.Cu") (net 15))
 (segment (start 91.825 52.325) (end 93 53.5) (width 0.2) (layer "F.Cu") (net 15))
 (segment (start 97 54) (end 97 73.765) (width 0.2) (layer "F.Cu") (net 15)))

